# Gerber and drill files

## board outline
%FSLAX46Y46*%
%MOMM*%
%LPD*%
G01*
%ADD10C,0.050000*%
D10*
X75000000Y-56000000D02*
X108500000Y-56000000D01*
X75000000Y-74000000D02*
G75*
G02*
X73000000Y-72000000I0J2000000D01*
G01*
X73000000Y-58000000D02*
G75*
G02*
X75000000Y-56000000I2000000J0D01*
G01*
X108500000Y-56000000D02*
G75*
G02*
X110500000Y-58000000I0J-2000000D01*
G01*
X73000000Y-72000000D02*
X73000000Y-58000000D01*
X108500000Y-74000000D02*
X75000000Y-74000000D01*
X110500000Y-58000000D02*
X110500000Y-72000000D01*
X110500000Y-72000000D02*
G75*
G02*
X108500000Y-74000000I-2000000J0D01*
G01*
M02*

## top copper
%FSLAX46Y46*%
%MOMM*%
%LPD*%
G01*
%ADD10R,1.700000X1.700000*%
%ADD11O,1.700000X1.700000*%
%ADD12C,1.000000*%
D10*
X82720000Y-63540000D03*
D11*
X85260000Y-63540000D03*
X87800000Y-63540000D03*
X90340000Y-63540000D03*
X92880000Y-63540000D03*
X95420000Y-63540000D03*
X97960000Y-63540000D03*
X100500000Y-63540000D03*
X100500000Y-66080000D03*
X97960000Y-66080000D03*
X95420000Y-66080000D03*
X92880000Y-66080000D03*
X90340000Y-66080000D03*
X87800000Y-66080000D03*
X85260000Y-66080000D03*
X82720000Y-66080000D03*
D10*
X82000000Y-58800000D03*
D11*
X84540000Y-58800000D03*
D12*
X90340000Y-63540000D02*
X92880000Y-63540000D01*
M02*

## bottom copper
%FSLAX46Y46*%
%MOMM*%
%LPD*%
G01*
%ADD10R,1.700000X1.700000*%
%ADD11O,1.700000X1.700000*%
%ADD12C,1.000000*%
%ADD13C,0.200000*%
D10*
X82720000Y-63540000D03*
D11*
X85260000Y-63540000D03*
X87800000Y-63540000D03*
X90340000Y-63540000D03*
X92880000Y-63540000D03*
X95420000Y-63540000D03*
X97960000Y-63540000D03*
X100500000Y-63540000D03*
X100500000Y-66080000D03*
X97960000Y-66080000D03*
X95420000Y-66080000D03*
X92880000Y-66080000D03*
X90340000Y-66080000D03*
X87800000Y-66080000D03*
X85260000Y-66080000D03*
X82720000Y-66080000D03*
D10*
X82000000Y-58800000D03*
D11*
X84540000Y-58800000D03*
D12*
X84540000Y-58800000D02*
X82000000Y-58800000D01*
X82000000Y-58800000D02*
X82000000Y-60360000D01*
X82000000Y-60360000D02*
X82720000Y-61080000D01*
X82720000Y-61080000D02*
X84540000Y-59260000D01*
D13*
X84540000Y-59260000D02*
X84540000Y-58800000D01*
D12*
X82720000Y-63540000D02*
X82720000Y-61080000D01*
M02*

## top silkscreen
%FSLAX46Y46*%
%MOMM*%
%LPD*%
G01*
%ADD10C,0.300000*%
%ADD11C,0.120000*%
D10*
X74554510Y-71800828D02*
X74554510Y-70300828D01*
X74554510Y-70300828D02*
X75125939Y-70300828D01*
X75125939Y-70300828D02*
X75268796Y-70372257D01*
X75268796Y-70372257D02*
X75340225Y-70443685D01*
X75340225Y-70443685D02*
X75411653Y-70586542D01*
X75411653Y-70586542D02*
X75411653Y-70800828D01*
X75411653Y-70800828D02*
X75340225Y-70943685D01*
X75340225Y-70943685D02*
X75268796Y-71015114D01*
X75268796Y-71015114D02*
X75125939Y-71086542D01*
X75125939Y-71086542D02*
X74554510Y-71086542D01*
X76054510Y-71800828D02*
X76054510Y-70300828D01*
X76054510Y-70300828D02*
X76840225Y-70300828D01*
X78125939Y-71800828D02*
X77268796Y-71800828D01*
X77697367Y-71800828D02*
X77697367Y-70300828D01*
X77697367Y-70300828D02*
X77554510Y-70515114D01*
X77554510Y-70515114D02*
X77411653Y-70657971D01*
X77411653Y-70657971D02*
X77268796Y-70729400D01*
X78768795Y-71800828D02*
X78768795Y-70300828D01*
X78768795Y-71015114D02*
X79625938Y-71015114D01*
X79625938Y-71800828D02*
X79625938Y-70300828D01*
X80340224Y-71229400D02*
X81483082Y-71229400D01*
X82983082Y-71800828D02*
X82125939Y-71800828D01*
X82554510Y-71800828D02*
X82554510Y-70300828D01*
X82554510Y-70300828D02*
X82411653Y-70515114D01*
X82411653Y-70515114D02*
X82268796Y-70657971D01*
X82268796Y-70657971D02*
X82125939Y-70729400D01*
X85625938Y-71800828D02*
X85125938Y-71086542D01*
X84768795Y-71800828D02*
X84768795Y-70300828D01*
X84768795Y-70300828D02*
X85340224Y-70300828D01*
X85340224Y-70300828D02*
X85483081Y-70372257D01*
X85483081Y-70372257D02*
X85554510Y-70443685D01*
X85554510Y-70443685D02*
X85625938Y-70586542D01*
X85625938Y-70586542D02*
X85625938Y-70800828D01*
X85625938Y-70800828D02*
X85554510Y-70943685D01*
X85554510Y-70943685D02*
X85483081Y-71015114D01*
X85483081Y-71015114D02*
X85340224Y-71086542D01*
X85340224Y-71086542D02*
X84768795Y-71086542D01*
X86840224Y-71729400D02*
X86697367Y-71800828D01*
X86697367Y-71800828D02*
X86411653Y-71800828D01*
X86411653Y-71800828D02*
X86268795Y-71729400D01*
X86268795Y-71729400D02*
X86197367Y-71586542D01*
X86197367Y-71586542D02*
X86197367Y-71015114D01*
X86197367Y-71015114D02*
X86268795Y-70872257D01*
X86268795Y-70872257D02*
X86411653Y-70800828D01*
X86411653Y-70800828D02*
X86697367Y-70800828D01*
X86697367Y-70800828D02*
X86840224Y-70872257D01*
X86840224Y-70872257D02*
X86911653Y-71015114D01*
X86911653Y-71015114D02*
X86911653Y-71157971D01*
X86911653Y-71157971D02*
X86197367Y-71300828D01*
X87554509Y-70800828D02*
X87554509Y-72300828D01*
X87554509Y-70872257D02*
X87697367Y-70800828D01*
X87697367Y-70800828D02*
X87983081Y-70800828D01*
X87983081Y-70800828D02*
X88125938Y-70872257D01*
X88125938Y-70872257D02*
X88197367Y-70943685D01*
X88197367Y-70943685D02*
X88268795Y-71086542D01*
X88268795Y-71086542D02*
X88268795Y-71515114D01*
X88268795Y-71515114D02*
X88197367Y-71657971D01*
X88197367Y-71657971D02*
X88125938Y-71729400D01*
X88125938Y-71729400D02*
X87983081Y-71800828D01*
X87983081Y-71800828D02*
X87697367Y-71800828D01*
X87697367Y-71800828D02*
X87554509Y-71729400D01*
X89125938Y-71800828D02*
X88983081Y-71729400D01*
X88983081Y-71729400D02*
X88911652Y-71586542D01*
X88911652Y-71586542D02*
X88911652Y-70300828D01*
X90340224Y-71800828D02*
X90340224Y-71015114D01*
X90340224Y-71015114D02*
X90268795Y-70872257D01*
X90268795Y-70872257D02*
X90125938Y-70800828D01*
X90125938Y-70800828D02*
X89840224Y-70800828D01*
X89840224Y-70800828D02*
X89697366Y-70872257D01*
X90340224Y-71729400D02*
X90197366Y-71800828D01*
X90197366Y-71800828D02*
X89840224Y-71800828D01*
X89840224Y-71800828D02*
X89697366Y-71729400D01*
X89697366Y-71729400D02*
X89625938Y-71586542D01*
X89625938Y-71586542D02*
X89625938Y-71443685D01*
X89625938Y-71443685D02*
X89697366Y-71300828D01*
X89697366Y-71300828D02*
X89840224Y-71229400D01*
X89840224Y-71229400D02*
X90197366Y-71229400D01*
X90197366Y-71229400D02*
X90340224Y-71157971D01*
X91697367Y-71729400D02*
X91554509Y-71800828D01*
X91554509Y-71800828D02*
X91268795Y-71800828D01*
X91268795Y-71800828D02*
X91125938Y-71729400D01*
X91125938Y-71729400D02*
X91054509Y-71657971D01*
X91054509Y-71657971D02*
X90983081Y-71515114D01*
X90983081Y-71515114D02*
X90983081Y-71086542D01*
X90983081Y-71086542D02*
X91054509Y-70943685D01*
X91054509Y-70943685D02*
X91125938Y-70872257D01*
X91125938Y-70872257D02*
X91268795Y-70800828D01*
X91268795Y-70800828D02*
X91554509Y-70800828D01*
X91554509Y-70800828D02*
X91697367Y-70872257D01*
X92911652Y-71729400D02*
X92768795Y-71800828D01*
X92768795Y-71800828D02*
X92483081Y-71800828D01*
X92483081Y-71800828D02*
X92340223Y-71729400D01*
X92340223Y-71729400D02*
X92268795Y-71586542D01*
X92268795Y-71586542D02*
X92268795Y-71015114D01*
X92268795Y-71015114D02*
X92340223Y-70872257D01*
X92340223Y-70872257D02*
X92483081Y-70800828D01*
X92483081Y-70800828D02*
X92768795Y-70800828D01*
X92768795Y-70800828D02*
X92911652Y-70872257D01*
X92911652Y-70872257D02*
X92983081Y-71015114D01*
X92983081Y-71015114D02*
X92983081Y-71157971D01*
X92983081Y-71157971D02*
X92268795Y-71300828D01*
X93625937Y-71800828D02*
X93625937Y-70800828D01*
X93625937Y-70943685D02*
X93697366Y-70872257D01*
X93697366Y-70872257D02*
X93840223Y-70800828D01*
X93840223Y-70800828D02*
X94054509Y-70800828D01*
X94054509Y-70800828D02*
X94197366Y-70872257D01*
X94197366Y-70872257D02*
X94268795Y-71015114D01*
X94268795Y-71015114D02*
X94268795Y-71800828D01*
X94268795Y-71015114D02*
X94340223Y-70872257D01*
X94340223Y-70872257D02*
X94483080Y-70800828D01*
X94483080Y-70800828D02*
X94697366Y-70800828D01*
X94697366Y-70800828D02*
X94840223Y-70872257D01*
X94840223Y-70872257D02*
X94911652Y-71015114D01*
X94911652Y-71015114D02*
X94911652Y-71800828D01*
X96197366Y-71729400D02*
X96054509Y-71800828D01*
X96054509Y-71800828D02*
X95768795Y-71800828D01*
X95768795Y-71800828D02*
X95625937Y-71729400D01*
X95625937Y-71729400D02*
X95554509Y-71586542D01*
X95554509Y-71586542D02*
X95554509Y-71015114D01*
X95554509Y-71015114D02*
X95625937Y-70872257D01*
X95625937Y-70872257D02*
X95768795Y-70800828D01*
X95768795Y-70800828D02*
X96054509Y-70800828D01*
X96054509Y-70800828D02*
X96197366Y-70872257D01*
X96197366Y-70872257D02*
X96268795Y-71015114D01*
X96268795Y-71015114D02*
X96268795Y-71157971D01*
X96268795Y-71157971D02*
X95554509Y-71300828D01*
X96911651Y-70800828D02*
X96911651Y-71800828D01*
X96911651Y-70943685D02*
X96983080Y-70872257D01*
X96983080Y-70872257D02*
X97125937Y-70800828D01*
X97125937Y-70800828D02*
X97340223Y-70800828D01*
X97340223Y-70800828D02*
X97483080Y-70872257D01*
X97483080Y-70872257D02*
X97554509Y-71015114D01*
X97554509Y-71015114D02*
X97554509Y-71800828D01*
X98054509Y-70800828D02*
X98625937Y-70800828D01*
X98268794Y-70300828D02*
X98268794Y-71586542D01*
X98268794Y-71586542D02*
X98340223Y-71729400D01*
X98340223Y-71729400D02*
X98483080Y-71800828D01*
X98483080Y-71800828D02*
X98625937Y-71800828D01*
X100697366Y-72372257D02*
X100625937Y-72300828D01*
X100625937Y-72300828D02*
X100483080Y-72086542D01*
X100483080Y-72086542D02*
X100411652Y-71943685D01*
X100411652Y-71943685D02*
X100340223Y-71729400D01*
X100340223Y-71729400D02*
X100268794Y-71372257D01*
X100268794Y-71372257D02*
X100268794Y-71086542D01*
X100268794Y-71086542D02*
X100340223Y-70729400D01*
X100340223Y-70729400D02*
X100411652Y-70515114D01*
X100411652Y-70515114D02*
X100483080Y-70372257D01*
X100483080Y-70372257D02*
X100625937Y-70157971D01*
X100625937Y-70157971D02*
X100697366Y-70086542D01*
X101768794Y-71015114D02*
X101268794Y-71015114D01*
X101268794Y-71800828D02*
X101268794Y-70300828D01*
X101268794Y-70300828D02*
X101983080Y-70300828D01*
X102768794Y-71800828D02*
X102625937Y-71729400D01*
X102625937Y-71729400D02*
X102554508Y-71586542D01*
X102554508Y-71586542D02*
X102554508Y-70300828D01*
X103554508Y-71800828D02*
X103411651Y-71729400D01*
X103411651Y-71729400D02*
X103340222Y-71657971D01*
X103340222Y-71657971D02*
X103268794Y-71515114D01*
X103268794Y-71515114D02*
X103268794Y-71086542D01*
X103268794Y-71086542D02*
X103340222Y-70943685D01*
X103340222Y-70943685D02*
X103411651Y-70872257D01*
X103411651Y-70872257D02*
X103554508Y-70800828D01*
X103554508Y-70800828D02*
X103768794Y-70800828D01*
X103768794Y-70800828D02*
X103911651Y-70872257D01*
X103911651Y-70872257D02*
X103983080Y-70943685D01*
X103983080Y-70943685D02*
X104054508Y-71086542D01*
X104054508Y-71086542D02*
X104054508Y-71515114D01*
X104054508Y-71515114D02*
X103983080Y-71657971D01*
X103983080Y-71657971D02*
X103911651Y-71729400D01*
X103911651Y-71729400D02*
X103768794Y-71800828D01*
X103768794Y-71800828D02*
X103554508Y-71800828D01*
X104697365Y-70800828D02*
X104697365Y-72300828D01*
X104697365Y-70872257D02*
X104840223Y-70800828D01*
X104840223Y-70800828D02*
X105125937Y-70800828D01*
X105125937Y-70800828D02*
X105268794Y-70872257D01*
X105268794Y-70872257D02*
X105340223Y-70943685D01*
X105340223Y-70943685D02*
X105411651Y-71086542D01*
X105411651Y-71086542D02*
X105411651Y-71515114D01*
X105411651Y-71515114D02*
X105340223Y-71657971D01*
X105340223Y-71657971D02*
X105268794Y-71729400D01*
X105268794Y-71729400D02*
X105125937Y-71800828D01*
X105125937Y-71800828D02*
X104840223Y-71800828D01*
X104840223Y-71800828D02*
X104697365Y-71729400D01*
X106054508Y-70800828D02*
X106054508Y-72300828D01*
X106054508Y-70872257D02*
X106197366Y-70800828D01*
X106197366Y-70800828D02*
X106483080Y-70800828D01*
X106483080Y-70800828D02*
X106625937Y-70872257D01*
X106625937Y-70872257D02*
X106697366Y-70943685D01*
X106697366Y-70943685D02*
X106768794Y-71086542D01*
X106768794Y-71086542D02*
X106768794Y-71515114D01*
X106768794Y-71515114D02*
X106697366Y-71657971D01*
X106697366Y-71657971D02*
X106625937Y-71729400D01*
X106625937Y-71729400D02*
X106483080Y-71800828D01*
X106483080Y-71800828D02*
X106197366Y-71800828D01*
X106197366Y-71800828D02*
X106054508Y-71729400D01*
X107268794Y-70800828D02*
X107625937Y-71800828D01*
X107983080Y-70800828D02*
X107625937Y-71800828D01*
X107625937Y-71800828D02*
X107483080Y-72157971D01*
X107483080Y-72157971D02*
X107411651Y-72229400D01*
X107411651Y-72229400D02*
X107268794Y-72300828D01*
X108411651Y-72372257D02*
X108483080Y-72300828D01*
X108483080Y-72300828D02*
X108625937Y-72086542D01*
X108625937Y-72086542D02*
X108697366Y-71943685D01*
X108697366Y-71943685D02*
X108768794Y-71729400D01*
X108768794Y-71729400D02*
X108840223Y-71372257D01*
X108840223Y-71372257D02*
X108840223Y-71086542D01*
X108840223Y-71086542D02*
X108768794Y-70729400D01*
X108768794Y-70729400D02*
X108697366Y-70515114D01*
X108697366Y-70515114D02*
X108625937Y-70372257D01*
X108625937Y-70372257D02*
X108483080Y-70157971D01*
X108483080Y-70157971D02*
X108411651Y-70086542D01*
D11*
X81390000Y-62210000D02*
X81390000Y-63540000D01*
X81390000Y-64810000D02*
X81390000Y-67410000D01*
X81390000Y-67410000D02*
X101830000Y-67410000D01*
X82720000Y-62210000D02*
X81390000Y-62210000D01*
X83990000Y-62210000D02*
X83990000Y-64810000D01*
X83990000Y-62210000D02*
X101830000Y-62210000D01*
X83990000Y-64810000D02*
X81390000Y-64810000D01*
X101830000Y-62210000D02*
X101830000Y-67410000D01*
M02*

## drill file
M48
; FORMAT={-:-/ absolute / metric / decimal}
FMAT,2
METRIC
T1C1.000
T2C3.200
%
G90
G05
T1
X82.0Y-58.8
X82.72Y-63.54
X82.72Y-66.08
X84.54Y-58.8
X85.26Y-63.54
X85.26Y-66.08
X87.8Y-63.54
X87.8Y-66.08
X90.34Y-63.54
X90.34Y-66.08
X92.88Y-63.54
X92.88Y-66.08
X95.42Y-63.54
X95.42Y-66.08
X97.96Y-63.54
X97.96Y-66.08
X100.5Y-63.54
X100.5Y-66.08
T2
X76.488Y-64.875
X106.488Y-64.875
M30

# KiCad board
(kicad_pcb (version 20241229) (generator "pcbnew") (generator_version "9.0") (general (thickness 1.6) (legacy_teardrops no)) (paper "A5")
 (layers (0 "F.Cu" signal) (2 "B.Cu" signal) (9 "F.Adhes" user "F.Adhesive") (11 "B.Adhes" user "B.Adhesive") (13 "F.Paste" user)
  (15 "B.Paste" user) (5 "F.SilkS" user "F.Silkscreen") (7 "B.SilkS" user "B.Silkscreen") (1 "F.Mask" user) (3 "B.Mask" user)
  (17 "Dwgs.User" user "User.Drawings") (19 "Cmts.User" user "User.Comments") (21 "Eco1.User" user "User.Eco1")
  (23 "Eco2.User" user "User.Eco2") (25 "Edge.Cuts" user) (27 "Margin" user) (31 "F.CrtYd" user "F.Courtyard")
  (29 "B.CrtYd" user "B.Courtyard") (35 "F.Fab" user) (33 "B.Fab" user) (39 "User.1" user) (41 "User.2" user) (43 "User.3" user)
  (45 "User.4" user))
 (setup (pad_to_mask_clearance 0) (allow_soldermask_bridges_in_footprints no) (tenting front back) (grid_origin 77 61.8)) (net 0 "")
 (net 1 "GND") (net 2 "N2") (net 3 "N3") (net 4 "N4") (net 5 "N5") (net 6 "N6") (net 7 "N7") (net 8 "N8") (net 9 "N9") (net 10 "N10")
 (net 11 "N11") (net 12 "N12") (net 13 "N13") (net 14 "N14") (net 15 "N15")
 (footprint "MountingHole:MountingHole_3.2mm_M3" (layer "F.Cu") (at 106.487631 64.875488)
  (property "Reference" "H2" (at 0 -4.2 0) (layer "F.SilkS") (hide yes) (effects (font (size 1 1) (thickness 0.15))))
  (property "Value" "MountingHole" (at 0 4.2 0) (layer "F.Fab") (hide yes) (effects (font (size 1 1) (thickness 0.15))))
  (pad "" np_thru_hole circle (at 0 0) (size 3.2 3.2) (drill 3.2) (layers "*.Cu" "*.Mask")))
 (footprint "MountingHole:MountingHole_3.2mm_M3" (layer "F.Cu") (at 76.487631 64.875488)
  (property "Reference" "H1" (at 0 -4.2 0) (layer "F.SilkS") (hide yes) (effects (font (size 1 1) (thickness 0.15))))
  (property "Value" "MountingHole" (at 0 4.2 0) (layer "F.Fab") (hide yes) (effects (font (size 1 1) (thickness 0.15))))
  (pad "" np_thru_hole circle (at 0 0) (size 3.2 3.2) (drill 3.2) (layers "*.Cu" "*.Mask")))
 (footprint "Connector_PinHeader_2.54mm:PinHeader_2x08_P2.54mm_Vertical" (layer "F.Cu") (at 82.72 65.54 90)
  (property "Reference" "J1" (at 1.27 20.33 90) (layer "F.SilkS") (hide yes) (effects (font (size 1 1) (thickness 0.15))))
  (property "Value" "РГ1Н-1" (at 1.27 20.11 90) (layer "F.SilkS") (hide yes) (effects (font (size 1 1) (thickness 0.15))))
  (fp_line (start 3.33 -1.33) (end 2 -1.33) (stroke (width 0.12) (type solid)) (layer "F.SilkS"))
  (fp_line (start 0.73 -1.33) (end -1.87 -1.33) (stroke (width 0.12) (type solid)) (layer "F.SilkS"))
  (fp_line (start -1.87 -1.33) (end -1.87 19.11) (stroke (width 0.12) (type solid)) (layer "F.SilkS"))
  (fp_line (start 3.33 0) (end 3.33 -1.33) (stroke (width 0.12) (type solid)) (layer "F.SilkS"))
  (fp_line (start 3.33 1.27) (end 0.73 1.27) (stroke (width 0.12) (type solid)) (layer "F.SilkS"))
  (fp_line (start 3.33 1.27) (end 3.33 19.11) (stroke (width 0.12) (type solid)) (layer "F.SilkS"))
  (fp_line (start 0.73 1.27) (end 0.73 -1.33) (stroke (width 0.12) (type solid)) (layer "F.SilkS"))
  (fp_line (start 3.33 19.11) (end -1.87 19.11) (stroke (width 0.12) (type solid)) (layer "F.SilkS"))
  (pad "1" thru_hole rect (at 2 0 90) (size 1.7 1.7) (drill 1) (layers "*.Cu" "*.Mask") (remove_unused_layers no) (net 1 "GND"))
  (pad "2" thru_hole oval (at 2 2.54 90) (size 1.7 1.7) (drill 1) (layers "*.Cu" "*.Mask") (remove_unused_layers no) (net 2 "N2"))
  (pad "3" thru_hole oval (at 2 5.08 90) (size 1.7 1.7) (drill 1) (layers "*.Cu" "*.Mask") (remove_unused_layers no) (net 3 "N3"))
  (pad "4" thru_hole oval (at 2 7.62 90) (size 1.7 1.7) (drill 1) (layers "*.Cu" "*.Mask") (remove_unused_layers no) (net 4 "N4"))
  (pad "5" thru_hole oval (at 2 10.16 90) (size 1.7 1.7) (drill 1) (layers "*.Cu" "*.Mask") (remove_unused_layers no) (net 4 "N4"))
  (pad "6" thru_hole oval (at 2 12.7 90) (size 1.7 1.7) (drill 1) (layers "*.Cu" "*.Mask") (remove_unused_layers no) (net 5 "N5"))
  (pad "7" thru_hole oval (at 2 15.24 90) (size 1.7 1.7) (drill 1) (layers "*.Cu" "*.Mask") (remove_unused_layers no) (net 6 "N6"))
  (pad "8" thru_hole oval (at 2 17.78 90) (size 1.7 1.7) (drill 1) (layers "*.Cu" "*.Mask") (remove_unused_layers no) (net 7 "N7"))
  (pad "9" thru_hole oval (at -0.54 17.78 90) (size 1.7 1.7) (drill 1) (layers "*.Cu" "*.Mask") (remove_unused_layers no) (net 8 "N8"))
  (pad "10" thru_hole oval (at -0.54 15.24 90) (size 1.7 1.7) (drill 1) (layers "*.Cu" "*.Mask") (remove_unused_layers no) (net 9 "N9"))
  (pad "11" thru_hole oval (at -0.54 12.7 90) (size 1.7 1.7) (drill 1) (layers "*.Cu" "*.Mask") (remove_unused_layers no) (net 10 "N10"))
  (pad "12" thru_hole oval (at -0.54 10.16 90) (size 1.7 1.7) (drill 1) (layers "*.Cu" "*.Mask") (remove_unused_layers no) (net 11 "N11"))
  (pad "13" thru_hole oval (at -0.54 7.62 90) (size 1.7 1.7) (drill 1) (layers "*.Cu" "*.Mask") (remove_unused_layers no) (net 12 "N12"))
  (pad "14" thru_hole oval (at -0.54 5.08 90) (size 1.7 1.7) (drill 1) (layers "*.Cu" "*.Mask") (remove_unused_layers no) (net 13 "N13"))
  (pad "15" thru_hole oval (at -0.54 2.54 90) (size 1.7 1.7) (drill 1) (layers "*.Cu" "*.Mask") (remove_unused_layers no) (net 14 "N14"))
  (pad "16" thru_hole oval (at -0.54 0 90) (size 1.7 1.7) (drill 1) (layers "*.Cu" "*.Mask") (remove_unused_layers no) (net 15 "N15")))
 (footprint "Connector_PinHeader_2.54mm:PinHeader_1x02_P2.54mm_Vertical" (layer "B.Cu") (at 82 58.8 -90)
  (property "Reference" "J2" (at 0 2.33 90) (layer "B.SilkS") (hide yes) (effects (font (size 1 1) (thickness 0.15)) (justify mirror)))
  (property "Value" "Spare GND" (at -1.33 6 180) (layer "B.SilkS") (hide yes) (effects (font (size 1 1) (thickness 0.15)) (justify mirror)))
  (pad "1" thru_hole rect (at 0 0 270) (size 1.7 1.7) (drill 1) (layers "*.Cu" "*.Mask") (remove_unused_layers no) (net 1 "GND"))
  (pad "2" thru_hole oval (at 0 -2.54 270) (size 1.7 1.7) (drill 1) (layers "*.Cu" "*.Mask") (remove_unused_layers no) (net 1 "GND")))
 (gr_line (start 75 56) (end 108.5 56) (stroke (width 0.05) (type default)) (layer "Edge.Cuts"))
 (gr_arc (start 75 74) (mid 73.585786 73.414214) (end 73 72) (stroke (width 0.05) (type default)) (layer "Edge.Cuts"))
 (gr_arc (start 73 58) (mid 73.585786 56.585786) (end 75 56) (stroke (width 0.05) (type default)) (layer "Edge.Cuts"))
 (gr_arc (start 108.5 56) (mid 109.914214 56.585786) (end 110.5 58) (stroke (width 0.05) (type default)) (layer "Edge.Cuts"))
 (gr_line (start 73 72) (end 73 58) (stroke (width 0.05) (type default)) (layer "Edge.Cuts"))
 (gr_line (start 108.5 74) (end 75 74) (stroke (width 0.05) (type default)) (layer "Edge.Cuts"))
 (gr_line (start 110.5 58) (end 110.5 72) (stroke (width 0.05) (type default)) (layer "Edge.Cuts"))
 (gr_arc (start 110.5 72) (mid 109.914214 73.414214) (end 108.5 74) (stroke (width 0.05) (type default)) (layer "Edge.Cuts"))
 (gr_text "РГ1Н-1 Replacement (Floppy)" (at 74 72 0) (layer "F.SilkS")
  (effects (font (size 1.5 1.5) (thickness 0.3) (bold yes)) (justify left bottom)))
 (segment (start 90.34 63.54) (end 92.88 63.54) (width 1) (layer "F.Cu") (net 4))
 (segment (start 84.54 58.8) (end 82 58.8) (width 1) (layer "B.Cu") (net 1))
 (segment (start 82 58.8) (end 82 60.36) (width 1) (layer "B.Cu") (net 1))
 (segment (start 82 60.36) (end 82.72 61.08) (width 1) (layer "B.Cu") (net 1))
 (segment (start 82.72 61.08) (end 84.54 59.26) (width 1) (layer "B.Cu") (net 1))
 (segment (start 84.54 59.26) (end 84.54 58.8) (width 0.2) (layer "B.Cu") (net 1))
 (segment (start 82.72 63.54) (end 82.72 61.08) (width 1) (layer "B.Cu") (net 1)))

